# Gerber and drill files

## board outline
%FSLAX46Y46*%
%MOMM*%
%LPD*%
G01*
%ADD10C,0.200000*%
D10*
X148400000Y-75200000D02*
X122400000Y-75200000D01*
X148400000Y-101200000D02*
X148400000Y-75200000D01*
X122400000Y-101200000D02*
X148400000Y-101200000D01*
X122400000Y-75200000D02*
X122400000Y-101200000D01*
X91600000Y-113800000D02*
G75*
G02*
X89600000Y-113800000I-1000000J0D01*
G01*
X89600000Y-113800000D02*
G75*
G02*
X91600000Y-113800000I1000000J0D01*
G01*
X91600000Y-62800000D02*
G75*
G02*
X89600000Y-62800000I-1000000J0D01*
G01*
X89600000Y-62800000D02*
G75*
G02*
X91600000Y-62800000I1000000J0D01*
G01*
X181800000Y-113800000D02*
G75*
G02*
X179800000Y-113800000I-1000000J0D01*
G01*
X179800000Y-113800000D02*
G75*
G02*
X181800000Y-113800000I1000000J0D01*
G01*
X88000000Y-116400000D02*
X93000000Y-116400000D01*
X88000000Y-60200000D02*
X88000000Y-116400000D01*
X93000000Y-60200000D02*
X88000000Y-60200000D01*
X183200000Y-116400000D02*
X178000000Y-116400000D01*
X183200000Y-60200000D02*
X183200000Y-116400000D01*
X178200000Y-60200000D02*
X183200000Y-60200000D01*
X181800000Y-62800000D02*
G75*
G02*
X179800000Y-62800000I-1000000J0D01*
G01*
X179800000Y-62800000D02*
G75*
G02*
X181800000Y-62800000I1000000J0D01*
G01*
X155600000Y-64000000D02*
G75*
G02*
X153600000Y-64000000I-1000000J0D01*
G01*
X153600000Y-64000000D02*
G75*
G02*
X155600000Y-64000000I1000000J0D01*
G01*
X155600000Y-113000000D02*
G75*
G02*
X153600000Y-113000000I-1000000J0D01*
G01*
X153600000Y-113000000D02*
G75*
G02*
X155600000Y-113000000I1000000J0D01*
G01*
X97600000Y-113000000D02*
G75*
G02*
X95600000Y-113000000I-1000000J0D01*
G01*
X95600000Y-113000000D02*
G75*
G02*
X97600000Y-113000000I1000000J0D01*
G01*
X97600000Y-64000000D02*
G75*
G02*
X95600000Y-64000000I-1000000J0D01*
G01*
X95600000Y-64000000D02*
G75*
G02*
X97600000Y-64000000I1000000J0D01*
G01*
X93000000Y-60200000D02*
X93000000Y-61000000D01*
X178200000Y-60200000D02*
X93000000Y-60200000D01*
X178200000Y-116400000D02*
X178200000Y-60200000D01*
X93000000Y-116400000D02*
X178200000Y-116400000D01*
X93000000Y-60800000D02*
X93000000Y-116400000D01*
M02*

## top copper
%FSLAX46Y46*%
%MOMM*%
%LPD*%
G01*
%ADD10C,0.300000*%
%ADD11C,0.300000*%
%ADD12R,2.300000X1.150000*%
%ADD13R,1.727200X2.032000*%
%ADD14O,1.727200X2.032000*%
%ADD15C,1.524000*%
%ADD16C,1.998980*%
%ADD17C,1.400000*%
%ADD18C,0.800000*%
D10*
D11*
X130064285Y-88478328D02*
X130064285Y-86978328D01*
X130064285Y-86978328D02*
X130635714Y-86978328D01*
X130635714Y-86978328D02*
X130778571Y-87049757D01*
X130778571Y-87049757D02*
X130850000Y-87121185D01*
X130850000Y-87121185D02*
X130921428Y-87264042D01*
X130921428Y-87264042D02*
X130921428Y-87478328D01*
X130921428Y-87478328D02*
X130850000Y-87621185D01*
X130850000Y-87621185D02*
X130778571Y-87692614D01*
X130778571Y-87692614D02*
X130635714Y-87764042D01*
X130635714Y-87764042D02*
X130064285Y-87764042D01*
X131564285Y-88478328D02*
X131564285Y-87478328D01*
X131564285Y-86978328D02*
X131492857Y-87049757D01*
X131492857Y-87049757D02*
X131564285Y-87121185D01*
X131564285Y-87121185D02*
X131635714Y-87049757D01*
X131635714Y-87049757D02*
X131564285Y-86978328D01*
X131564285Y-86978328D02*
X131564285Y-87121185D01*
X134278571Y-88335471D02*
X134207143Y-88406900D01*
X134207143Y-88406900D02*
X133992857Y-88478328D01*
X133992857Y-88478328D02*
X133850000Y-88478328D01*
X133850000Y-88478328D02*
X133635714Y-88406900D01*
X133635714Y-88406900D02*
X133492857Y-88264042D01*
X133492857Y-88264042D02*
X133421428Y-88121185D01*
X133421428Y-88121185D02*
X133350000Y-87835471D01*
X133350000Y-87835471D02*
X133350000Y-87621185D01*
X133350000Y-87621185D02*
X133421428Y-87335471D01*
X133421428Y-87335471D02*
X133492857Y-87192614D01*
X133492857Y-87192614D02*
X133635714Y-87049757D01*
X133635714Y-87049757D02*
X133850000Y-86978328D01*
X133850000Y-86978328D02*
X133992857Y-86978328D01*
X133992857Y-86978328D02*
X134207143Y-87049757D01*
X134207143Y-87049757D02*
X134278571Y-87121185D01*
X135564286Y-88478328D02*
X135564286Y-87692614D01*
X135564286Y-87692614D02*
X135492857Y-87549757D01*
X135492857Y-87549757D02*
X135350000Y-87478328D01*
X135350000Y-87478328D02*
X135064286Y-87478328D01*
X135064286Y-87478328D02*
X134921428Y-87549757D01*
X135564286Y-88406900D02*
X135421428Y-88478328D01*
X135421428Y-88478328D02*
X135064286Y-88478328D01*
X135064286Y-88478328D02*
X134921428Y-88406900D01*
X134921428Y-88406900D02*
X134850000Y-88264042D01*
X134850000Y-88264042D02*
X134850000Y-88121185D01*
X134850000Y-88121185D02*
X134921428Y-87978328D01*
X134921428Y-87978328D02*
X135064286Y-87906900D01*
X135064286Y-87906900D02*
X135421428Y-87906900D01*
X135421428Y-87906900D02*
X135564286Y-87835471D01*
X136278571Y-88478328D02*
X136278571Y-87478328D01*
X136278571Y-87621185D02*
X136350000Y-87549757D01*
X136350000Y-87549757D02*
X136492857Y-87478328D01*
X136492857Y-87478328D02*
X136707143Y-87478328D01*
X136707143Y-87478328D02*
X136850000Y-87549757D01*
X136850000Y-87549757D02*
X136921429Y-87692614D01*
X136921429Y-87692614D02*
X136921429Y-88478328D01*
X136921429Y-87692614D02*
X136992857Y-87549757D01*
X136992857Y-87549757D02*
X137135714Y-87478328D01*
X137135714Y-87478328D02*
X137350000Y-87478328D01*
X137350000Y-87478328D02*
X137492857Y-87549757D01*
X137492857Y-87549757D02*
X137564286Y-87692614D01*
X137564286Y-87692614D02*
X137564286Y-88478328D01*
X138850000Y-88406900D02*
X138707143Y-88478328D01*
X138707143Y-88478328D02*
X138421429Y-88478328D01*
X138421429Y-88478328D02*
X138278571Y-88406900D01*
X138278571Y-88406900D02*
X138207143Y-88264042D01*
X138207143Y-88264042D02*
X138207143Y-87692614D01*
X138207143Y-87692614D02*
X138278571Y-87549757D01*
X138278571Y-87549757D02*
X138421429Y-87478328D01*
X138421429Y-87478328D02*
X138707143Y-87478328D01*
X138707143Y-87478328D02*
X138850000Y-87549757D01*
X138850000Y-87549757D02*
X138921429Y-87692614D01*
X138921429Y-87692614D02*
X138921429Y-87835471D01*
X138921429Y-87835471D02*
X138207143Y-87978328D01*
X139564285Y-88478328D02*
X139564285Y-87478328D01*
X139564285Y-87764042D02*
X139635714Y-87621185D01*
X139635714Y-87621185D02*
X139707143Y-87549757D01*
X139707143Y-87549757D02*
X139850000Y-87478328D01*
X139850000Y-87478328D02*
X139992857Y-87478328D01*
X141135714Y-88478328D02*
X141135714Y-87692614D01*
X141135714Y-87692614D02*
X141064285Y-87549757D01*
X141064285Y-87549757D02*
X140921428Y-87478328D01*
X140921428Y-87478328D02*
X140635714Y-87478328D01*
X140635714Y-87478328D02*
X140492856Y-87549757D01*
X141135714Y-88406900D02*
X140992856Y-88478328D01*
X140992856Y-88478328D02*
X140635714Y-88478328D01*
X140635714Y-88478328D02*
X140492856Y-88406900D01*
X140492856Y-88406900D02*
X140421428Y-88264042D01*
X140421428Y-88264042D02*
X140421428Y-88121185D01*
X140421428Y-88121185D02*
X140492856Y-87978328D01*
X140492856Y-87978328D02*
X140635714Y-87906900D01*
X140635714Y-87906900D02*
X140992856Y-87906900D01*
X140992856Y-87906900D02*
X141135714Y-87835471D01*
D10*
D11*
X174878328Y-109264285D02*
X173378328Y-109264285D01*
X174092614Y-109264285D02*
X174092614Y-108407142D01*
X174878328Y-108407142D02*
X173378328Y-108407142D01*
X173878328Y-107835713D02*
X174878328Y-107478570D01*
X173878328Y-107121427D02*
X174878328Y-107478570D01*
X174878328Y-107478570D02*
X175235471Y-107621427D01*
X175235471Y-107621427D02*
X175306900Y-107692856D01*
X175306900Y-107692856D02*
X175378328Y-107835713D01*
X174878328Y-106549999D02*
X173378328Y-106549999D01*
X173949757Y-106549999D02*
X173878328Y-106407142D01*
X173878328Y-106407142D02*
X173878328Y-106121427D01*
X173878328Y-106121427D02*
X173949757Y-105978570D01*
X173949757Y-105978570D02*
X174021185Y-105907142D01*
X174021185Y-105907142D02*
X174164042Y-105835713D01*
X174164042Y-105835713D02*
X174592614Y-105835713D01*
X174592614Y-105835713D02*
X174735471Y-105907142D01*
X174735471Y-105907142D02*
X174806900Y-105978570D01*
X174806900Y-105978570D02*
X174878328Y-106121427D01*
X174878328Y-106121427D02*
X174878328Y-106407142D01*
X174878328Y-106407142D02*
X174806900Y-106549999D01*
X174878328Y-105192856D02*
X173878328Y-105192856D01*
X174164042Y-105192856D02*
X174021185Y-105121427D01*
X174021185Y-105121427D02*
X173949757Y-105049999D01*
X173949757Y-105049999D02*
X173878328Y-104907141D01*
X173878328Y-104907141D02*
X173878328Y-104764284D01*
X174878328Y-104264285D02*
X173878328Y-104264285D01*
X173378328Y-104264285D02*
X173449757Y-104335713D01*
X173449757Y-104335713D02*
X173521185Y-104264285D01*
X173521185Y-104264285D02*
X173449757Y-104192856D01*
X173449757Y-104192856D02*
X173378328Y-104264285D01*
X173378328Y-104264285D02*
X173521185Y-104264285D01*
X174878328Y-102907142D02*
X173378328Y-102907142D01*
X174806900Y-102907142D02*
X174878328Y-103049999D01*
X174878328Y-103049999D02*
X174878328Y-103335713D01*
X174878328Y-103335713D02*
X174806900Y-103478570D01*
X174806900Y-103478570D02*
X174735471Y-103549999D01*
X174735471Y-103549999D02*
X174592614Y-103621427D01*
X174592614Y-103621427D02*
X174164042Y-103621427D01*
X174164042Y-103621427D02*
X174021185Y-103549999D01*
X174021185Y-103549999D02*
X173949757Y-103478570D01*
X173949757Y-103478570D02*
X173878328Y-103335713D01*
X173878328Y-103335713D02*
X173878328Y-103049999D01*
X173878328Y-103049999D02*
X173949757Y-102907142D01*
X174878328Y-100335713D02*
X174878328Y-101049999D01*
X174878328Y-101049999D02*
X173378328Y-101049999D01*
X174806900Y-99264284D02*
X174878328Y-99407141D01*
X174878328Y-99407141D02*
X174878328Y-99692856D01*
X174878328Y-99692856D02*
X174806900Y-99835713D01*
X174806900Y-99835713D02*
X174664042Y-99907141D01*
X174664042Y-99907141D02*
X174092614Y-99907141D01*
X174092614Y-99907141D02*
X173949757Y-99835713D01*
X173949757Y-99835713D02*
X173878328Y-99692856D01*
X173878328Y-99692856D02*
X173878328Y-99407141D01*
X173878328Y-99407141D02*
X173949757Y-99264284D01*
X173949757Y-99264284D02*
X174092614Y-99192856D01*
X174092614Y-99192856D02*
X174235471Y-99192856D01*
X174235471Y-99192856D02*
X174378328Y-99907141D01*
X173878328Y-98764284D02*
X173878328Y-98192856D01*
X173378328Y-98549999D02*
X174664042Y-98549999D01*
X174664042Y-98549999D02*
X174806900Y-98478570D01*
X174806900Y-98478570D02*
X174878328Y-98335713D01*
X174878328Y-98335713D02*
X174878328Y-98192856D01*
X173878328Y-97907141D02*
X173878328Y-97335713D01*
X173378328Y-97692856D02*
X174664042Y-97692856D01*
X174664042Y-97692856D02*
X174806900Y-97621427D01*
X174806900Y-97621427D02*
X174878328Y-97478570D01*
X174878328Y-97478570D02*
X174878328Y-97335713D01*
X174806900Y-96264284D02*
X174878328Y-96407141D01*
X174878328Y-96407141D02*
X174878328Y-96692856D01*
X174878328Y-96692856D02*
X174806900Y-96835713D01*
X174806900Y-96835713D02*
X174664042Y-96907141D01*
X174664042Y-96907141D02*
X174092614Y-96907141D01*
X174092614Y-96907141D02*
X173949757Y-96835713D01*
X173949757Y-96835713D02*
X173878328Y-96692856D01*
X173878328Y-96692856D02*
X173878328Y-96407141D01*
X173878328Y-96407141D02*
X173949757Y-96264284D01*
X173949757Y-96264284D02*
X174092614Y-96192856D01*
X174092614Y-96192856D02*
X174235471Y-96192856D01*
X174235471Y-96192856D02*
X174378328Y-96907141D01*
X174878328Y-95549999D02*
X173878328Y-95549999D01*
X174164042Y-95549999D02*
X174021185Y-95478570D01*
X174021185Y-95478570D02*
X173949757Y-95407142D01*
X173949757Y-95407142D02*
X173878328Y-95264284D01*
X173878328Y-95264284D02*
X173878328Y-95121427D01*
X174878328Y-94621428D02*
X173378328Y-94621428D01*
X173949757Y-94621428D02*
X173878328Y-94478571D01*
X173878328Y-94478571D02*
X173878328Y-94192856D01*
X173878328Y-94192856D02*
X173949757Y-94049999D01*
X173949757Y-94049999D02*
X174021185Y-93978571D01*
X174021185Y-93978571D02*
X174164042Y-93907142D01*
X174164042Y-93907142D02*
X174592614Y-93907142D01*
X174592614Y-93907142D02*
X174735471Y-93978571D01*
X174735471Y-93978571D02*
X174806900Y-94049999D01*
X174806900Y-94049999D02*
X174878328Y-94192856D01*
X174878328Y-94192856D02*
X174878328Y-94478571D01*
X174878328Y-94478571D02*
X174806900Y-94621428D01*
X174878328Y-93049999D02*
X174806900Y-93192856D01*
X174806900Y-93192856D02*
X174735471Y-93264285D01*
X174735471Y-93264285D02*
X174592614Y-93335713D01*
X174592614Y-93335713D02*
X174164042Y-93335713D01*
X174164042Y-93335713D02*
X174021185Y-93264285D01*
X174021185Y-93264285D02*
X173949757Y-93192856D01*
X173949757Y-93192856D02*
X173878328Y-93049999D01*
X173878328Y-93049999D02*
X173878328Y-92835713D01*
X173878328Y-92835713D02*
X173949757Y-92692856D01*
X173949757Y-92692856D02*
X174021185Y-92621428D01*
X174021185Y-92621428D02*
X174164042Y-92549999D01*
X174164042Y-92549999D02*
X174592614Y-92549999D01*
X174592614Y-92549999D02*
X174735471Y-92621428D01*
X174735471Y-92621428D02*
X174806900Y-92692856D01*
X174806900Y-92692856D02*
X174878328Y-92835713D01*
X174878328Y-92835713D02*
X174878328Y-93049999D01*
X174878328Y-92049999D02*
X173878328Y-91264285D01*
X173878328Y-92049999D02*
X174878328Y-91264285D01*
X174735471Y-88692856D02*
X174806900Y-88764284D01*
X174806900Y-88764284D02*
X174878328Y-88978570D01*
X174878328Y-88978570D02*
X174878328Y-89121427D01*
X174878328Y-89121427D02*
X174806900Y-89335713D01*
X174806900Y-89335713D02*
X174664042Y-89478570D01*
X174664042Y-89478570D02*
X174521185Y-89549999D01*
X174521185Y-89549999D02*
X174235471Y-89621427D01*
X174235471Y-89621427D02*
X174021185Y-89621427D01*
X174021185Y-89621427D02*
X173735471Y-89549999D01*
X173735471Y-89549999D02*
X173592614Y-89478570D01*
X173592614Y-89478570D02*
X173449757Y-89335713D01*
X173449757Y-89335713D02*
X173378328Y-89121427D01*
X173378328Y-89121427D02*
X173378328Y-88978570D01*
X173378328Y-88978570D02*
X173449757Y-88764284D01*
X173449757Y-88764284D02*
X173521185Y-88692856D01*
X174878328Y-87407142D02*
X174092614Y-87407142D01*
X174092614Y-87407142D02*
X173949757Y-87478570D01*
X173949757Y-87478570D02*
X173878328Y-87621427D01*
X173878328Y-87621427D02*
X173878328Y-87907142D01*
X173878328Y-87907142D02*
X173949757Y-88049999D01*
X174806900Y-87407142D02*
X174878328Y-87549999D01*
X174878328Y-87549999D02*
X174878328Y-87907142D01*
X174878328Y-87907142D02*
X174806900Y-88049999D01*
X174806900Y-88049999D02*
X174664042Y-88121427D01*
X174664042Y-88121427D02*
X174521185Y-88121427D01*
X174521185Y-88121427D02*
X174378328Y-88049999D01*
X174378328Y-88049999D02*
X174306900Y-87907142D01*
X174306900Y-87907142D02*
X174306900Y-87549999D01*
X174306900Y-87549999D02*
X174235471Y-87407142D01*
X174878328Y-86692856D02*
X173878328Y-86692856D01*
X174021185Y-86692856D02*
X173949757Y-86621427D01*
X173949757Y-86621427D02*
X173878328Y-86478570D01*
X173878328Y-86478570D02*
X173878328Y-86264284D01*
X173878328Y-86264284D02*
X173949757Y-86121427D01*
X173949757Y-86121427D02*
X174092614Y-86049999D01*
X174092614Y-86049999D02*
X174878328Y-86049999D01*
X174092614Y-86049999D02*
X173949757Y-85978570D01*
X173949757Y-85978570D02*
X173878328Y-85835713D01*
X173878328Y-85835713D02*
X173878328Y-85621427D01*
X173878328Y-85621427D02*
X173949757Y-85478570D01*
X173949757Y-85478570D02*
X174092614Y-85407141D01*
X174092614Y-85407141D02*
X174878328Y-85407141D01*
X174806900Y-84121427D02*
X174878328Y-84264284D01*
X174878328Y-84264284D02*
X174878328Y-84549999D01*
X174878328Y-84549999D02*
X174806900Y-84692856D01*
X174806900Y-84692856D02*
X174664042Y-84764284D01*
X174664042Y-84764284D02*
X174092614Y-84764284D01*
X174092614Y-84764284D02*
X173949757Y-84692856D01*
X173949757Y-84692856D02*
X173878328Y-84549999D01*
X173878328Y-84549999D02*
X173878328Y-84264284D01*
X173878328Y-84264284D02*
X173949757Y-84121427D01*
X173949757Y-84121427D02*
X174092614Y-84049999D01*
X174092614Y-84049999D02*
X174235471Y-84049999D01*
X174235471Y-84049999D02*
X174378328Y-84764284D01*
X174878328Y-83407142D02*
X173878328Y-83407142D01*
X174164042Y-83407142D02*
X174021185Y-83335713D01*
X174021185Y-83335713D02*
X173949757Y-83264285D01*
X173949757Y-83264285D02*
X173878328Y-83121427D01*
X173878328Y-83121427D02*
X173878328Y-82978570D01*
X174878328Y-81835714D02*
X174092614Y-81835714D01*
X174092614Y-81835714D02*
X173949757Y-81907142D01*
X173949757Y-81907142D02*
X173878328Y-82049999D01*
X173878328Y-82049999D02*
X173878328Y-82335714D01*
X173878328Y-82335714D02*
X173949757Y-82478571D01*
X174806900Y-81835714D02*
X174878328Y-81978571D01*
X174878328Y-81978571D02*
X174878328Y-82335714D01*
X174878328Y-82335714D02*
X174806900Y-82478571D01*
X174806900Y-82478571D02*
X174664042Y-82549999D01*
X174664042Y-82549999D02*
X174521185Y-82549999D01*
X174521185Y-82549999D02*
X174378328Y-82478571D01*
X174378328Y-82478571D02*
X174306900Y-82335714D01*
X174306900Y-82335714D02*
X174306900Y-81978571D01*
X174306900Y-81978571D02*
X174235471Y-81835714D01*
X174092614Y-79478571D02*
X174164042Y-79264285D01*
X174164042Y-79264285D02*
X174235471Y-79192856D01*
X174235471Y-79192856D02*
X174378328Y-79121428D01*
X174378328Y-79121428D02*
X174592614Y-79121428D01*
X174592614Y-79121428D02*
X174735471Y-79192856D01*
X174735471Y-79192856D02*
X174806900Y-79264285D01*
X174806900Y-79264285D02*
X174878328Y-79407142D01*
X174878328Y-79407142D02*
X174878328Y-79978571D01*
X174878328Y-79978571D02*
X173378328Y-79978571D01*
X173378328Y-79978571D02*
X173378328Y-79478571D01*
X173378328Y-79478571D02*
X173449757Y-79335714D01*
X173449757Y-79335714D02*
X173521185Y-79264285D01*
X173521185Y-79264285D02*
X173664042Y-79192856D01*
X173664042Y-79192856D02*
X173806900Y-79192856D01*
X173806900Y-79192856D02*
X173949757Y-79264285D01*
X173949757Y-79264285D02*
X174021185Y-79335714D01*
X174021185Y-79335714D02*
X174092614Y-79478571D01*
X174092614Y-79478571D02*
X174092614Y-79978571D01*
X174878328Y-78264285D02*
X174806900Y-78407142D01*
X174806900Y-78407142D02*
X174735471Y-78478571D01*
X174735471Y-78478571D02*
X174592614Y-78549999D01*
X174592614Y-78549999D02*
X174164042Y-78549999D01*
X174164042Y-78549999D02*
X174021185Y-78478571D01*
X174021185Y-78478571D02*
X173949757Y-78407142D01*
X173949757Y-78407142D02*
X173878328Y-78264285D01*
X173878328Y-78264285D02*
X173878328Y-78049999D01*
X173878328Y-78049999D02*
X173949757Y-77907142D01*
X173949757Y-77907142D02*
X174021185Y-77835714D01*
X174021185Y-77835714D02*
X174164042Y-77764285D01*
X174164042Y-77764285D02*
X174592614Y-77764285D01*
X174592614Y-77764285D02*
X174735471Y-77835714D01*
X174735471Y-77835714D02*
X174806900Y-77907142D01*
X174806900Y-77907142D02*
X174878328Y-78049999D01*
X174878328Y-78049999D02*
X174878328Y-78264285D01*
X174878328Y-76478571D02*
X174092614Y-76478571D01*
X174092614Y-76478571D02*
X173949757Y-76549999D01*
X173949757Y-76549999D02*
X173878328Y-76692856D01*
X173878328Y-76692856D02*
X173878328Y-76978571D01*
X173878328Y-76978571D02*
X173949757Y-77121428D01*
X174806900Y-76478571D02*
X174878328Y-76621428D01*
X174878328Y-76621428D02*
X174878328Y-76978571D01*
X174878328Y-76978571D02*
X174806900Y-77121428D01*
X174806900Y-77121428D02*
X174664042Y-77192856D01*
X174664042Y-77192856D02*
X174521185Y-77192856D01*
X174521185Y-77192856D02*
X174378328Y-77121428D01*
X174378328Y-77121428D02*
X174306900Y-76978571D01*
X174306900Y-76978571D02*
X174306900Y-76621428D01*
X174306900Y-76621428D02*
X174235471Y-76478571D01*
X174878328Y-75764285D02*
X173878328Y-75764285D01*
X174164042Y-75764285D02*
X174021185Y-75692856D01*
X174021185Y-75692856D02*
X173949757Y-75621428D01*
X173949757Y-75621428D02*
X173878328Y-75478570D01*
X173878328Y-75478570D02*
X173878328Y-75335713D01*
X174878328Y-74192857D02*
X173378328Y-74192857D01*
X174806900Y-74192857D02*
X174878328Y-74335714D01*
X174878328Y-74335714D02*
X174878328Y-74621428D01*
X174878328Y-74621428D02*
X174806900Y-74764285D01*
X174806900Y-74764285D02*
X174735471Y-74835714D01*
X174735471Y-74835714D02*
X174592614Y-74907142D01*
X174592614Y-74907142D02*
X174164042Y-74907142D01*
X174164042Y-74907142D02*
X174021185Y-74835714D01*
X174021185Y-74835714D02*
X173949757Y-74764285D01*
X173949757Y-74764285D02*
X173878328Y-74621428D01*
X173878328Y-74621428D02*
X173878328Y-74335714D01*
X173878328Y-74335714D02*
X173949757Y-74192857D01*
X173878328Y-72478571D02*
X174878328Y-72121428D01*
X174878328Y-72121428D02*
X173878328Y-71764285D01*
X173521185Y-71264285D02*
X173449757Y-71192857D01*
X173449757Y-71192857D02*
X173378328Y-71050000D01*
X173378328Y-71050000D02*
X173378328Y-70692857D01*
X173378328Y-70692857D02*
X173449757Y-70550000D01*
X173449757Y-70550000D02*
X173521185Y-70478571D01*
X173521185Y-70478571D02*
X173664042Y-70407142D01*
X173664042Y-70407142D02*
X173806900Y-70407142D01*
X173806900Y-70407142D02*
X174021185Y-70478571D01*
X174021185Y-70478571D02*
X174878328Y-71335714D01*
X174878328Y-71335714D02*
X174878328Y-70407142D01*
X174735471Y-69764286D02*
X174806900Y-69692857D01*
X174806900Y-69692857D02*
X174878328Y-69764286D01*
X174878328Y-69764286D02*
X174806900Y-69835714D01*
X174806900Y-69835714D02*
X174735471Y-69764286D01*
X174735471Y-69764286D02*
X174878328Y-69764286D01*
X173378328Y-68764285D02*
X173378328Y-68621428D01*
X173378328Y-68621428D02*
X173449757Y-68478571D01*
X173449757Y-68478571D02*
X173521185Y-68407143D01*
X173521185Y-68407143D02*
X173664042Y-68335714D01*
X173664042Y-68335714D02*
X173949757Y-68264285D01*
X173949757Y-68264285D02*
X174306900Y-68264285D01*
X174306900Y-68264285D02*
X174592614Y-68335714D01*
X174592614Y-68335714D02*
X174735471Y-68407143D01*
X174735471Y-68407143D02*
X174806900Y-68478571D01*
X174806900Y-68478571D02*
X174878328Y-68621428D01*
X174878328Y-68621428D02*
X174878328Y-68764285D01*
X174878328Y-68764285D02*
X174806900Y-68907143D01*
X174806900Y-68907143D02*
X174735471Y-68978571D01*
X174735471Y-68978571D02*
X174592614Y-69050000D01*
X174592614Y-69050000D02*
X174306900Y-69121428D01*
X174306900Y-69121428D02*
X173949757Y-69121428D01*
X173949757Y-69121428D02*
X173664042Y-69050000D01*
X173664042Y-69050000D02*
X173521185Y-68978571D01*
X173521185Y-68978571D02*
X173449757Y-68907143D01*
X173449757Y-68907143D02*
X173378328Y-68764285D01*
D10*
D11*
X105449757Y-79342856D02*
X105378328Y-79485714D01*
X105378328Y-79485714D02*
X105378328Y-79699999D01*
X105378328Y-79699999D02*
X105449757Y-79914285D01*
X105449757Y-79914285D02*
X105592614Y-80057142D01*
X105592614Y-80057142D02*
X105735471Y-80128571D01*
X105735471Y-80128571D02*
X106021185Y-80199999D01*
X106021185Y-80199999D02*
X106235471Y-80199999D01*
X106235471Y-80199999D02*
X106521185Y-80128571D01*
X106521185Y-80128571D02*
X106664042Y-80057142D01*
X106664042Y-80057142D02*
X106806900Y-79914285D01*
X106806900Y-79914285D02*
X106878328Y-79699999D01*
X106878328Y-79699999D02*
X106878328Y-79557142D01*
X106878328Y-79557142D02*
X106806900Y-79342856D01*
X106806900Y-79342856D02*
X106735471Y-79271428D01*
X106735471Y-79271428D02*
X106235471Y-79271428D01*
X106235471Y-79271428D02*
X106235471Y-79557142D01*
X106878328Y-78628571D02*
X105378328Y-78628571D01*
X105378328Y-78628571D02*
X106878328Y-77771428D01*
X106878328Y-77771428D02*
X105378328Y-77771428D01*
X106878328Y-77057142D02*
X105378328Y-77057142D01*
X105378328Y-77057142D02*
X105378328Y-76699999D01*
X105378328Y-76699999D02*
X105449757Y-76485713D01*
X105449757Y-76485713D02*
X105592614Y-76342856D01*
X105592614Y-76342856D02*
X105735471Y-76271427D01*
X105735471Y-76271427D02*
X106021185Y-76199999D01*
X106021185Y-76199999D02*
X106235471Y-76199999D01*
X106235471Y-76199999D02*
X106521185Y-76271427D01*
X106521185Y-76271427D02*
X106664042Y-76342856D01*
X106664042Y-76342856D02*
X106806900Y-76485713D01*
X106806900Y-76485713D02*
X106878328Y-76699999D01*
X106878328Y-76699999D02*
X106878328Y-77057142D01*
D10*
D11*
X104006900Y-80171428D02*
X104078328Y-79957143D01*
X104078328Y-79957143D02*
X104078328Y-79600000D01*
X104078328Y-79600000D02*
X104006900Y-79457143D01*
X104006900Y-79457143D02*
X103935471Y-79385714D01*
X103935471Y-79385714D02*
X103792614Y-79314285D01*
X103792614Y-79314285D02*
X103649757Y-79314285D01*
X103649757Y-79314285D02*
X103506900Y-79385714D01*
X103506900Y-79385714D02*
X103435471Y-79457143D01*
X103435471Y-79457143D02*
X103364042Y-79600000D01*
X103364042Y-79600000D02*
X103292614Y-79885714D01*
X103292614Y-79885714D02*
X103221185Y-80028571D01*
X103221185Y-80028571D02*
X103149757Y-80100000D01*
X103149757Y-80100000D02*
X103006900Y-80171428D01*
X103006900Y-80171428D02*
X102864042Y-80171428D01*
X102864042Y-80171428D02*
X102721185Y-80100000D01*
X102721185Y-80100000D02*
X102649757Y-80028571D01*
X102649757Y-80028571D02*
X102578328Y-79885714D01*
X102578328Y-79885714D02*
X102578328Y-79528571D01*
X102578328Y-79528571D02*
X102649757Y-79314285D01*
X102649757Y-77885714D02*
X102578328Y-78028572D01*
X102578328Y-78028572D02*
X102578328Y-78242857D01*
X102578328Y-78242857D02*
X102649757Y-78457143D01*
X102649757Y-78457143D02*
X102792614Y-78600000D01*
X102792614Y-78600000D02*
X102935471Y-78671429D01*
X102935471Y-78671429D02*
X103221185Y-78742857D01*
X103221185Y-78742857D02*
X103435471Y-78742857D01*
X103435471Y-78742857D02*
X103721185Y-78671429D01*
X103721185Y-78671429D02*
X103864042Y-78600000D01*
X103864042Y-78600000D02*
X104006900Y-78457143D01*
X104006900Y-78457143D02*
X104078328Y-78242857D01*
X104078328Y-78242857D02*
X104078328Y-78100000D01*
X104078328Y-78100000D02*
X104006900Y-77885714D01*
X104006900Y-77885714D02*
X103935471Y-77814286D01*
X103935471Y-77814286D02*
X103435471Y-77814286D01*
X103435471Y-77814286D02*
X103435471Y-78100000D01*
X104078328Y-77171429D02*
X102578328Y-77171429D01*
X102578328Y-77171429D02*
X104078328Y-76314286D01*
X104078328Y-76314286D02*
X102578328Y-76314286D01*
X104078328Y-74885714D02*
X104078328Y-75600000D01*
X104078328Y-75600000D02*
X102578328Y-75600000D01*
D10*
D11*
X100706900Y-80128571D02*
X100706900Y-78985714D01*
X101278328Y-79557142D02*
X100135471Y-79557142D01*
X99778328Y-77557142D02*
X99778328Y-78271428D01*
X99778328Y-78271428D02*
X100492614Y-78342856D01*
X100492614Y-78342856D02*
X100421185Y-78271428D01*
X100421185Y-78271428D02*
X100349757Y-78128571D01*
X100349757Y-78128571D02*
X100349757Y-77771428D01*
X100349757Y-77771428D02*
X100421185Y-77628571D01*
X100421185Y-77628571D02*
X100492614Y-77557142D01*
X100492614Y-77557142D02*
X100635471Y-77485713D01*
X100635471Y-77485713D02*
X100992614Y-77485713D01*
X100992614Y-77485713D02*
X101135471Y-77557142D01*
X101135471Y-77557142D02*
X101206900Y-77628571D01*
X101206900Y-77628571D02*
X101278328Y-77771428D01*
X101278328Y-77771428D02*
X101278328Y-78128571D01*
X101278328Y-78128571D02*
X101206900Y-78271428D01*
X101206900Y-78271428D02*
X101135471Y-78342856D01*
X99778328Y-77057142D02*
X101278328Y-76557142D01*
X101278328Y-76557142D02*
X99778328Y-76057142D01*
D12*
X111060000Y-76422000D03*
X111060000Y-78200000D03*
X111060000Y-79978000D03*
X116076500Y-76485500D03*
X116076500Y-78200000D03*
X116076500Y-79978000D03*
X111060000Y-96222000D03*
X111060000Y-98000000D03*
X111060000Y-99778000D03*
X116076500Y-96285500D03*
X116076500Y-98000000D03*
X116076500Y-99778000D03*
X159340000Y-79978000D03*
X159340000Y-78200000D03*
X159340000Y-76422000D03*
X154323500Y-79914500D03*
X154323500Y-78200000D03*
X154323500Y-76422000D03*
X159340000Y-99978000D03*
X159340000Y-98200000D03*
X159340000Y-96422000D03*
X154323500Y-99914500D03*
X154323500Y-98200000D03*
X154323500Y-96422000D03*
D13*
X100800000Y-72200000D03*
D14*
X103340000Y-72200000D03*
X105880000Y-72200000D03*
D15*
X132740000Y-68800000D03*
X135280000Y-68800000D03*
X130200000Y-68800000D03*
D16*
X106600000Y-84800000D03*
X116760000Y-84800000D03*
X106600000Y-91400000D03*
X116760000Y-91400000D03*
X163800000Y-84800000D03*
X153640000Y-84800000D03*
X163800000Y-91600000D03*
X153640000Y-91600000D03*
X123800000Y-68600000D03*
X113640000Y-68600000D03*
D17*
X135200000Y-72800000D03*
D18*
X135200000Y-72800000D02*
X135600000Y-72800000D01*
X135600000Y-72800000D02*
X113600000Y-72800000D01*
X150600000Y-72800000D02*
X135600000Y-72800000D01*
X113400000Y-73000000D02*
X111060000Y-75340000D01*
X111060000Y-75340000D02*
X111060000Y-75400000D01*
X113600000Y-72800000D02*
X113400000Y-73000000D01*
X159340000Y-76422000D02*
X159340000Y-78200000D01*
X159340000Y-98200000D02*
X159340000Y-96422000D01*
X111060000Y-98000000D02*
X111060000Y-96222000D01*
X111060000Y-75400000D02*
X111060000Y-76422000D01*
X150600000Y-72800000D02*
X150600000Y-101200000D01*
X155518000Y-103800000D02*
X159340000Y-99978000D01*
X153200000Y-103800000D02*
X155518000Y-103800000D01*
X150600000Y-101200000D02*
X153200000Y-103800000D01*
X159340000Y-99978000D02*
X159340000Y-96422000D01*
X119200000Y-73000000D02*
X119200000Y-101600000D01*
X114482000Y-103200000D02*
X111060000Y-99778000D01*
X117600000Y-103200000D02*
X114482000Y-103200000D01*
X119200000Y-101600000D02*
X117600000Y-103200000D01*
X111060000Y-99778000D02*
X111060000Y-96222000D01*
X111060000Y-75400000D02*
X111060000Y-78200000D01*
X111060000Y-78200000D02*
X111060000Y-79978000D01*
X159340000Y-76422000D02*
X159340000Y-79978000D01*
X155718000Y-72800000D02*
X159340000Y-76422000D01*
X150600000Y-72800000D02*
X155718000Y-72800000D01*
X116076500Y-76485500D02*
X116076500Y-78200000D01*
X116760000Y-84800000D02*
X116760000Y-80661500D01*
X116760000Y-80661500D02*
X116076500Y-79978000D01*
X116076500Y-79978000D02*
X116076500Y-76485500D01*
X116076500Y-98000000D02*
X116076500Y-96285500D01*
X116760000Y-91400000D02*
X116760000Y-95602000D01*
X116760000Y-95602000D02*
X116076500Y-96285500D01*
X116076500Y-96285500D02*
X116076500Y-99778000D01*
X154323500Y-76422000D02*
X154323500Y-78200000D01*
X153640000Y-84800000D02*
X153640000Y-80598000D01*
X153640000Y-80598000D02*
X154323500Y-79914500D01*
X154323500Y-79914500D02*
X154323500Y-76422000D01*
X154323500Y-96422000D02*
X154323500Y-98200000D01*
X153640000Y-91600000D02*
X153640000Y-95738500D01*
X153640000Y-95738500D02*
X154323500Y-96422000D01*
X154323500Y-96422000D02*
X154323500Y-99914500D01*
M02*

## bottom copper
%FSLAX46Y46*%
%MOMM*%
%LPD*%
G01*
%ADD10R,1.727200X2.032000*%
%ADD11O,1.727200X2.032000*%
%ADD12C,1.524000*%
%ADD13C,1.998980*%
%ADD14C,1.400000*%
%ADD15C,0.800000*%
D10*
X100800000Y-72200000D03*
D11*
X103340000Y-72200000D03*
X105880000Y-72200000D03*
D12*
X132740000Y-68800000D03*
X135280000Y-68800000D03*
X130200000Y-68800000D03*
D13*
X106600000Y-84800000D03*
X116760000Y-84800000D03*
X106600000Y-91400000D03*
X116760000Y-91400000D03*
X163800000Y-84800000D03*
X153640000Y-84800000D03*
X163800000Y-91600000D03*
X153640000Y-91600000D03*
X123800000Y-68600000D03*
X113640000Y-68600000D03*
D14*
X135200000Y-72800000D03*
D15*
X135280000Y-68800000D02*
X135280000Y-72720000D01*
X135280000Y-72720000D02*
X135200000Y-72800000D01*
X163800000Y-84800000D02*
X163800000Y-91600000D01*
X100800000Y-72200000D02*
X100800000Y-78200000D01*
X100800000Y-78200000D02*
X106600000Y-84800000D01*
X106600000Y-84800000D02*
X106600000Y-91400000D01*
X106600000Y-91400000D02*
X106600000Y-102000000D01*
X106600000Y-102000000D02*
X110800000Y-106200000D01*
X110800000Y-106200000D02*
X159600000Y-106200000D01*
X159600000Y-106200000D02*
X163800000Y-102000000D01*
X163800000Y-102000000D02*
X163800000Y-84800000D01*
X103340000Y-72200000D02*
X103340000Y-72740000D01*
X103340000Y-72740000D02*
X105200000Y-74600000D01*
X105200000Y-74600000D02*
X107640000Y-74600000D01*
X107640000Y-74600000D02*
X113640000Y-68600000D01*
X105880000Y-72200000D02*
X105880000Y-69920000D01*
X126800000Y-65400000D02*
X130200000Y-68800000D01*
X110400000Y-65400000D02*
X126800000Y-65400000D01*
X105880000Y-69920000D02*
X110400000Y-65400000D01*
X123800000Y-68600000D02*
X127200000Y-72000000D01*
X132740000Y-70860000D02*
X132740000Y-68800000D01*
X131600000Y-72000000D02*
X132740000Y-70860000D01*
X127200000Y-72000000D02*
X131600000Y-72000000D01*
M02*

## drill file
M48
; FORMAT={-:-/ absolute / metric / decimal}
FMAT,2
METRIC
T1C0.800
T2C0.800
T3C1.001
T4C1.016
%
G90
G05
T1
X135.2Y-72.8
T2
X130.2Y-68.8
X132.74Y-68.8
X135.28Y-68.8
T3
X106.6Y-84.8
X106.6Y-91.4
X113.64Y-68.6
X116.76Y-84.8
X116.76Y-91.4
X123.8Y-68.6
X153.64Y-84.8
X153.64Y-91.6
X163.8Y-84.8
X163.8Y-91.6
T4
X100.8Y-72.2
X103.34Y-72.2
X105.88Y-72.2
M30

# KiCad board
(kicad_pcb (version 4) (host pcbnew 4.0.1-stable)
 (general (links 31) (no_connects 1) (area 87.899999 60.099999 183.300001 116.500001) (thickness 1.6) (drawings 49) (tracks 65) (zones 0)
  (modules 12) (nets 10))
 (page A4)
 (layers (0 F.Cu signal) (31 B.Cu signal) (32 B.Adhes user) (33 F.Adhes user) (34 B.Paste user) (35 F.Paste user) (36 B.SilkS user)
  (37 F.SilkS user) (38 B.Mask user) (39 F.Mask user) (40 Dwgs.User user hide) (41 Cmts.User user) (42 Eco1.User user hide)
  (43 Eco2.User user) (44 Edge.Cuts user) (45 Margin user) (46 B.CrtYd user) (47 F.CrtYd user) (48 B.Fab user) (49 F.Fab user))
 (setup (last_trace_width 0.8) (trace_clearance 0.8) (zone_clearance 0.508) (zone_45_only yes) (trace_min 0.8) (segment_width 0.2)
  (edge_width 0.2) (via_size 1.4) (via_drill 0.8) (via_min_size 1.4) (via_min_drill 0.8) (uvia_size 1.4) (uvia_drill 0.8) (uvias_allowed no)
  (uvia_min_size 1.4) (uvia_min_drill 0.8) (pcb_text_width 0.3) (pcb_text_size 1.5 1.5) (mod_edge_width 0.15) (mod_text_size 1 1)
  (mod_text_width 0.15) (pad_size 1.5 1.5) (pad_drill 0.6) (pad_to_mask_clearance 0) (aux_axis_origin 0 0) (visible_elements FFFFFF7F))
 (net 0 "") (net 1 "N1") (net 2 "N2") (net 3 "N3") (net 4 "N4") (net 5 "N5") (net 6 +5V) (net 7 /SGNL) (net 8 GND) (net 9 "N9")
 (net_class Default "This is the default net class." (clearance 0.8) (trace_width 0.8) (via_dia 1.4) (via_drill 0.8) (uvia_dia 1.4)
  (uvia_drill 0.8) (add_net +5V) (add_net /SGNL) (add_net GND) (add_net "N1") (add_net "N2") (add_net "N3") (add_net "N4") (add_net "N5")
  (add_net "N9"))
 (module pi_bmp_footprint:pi (layer F.Cu) (at 135.4 88.2)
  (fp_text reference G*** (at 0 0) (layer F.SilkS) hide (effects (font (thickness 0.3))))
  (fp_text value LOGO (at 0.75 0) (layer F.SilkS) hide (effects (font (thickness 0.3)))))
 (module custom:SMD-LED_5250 (layer F.Cu) (at 113.6 78.2)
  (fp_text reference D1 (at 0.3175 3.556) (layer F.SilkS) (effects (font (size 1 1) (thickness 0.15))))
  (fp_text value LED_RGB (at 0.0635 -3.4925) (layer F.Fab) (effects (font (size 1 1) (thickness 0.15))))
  (pad 1 smd rect (at -2.54 -1.778) (size 2.3 1.15) (layers F.Cu F.Paste F.Mask) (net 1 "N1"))
  (pad 2 smd rect (at -2.54 0) (size 2.3 1.15) (layers F.Cu F.Paste F.Mask) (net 1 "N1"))
  (pad 3 smd rect (at -2.54 1.778) (size 2.3 1.15) (layers F.Cu F.Paste F.Mask) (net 1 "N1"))
  (pad 4 smd rect (at 2.4765 -1.7145) (size 2.3 1.15) (layers F.Cu F.Paste F.Mask) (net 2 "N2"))
  (pad 5 smd rect (at 2.4765 0) (size 2.3 1.15) (layers F.Cu F.Paste F.Mask) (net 2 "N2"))
  (pad 6 smd rect (at 2.4765 1.778) (size 2.3 1.15) (layers F.Cu F.Paste F.Mask) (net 2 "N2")))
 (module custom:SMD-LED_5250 (layer F.Cu) (at 113.6 98)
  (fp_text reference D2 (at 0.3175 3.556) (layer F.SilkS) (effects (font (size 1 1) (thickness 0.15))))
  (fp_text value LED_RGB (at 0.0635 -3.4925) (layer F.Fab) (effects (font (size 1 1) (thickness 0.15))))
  (pad 1 smd rect (at -2.54 -1.778) (size 2.3 1.15) (layers F.Cu F.Paste F.Mask) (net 1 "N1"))
  (pad 2 smd rect (at -2.54 0) (size 2.3 1.15) (layers F.Cu F.Paste F.Mask) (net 1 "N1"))
  (pad 3 smd rect (at -2.54 1.778) (size 2.3 1.15) (layers F.Cu F.Paste F.Mask) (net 1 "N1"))
  (pad 4 smd rect (at 2.4765 -1.7145) (size 2.3 1.15) (layers F.Cu F.Paste F.Mask) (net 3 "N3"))
  (pad 5 smd rect (at 2.4765 0) (size 2.3 1.15) (layers F.Cu F.Paste F.Mask) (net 3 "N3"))
  (pad 6 smd rect (at 2.4765 1.778) (size 2.3 1.15) (layers F.Cu F.Paste F.Mask) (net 3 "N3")))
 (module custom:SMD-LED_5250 (layer F.Cu) (at 156.8 78.2 180)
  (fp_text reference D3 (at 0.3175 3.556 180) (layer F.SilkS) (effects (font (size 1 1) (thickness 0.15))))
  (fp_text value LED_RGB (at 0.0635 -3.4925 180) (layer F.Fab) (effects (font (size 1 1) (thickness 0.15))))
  (pad 1 smd rect (at -2.54 -1.778 180) (size 2.3 1.15) (layers F.Cu F.Paste F.Mask) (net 1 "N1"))
  (pad 2 smd rect (at -2.54 0 180) (size 2.3 1.15) (layers F.Cu F.Paste F.Mask) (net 1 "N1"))
  (pad 3 smd rect (at -2.54 1.778 180) (size 2.3 1.15) (layers F.Cu F.Paste F.Mask) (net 1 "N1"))
  (pad 4 smd rect (at 2.4765 -1.7145 180) (size 2.3 1.15) (layers F.Cu F.Paste F.Mask) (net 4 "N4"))
  (pad 5 smd rect (at 2.4765 0 180) (size 2.3 1.15) (layers F.Cu F.Paste F.Mask) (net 4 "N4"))
  (pad 6 smd rect (at 2.4765 1.778 180) (size 2.3 1.15) (layers F.Cu F.Paste F.Mask) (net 4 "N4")))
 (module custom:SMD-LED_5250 (layer F.Cu) (at 156.8 98.2 180)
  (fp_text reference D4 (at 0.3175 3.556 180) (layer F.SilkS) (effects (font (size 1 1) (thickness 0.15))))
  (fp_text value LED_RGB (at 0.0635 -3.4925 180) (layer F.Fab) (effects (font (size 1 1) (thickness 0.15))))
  (pad 1 smd rect (at -2.54 -1.778 180) (size 2.3 1.15) (layers F.Cu F.Paste F.Mask) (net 1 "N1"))
  (pad 2 smd rect (at -2.54 0 180) (size 2.3 1.15) (layers F.Cu F.Paste F.Mask) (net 1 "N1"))
  (pad 3 smd rect (at -2.54 1.778 180) (size 2.3 1.15) (layers F.Cu F.Paste F.Mask) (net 1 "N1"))
  (pad 4 smd rect (at 2.4765 -1.7145 180) (size 2.3 1.15) (layers F.Cu F.Paste F.Mask) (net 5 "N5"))
  (pad 5 smd rect (at 2.4765 0 180) (size 2.3 1.15) (layers F.Cu F.Paste F.Mask) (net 5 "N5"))
  (pad 6 smd rect (at 2.4765 1.778 180) (size 2.3 1.15) (layers F.Cu F.Paste F.Mask) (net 5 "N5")))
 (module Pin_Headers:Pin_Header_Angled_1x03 (layer F.Cu) (at 100.8 72.2 90)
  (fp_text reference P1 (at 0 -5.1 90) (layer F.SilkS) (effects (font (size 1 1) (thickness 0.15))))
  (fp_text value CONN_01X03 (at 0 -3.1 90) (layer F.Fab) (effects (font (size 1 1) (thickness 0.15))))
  (pad 1 thru_hole rect (at 0 0 90) (size 2.032 1.7272) (drill 1.016) (layers *.Cu *.Mask F.SilkS) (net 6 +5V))
  (pad 2 thru_hole oval (at 0 2.54 90) (size 2.032 1.7272) (drill 1.016) (layers *.Cu *.Mask F.SilkS) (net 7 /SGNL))
  (pad 3 thru_hole oval (at 0 5.08 90) (size 2.032 1.7272) (drill 1.016) (layers *.Cu *.Mask F.SilkS) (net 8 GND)))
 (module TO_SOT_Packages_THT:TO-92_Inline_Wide (layer F.Cu) (at 130.2 68.8)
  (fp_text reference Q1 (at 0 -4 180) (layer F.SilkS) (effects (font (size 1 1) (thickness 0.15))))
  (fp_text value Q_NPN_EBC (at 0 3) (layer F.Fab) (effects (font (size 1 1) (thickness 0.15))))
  (pad 2 thru_hole circle (at 2.54 0 90) (size 1.524 1.524) (drill 0.8) (layers *.Cu *.Mask F.SilkS) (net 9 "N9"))
  (pad 3 thru_hole circle (at 5.08 0 90) (size 1.524 1.524) (drill 0.8) (layers *.Cu *.Mask F.SilkS) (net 1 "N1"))
  (pad 1 thru_hole circle (at 0 0 90) (size 1.524 1.524) (drill 0.8) (layers *.Cu *.Mask F.SilkS) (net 8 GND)))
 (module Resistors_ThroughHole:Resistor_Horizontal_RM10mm (layer F.Cu) (at 106.6 84.8)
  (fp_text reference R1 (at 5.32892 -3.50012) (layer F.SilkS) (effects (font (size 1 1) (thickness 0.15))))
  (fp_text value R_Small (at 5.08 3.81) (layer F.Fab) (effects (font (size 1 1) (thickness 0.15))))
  (pad 1 thru_hole circle (at 0 0) (size 1.99898 1.99898) (drill 1.00076) (layers *.Cu *.SilkS *.Mask) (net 6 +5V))
  (pad 2 thru_hole circle (at 10.16 0) (size 1.99898 1.99898) (drill 1.00076) (layers *.Cu *.SilkS *.Mask) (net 2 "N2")))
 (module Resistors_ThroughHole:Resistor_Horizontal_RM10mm (layer F.Cu) (at 106.6 91.4)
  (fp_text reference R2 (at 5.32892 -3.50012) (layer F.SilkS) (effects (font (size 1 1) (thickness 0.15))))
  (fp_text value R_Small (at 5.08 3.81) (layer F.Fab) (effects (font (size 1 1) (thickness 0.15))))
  (pad 1 thru_hole circle (at 0 0) (size 1.99898 1.99898) (drill 1.00076) (layers *.Cu *.SilkS *.Mask) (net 6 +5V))
  (pad 2 thru_hole circle (at 10.16 0) (size 1.99898 1.99898) (drill 1.00076) (layers *.Cu *.SilkS *.Mask) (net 3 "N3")))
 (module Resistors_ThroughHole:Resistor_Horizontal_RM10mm (layer F.Cu) (at 163.8 84.8 180)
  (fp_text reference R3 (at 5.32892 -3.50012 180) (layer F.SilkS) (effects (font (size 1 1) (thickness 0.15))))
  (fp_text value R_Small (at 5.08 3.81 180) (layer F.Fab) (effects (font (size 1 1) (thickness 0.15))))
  (pad 1 thru_hole circle (at 0 0 180) (size 1.99898 1.99898) (drill 1.00076) (layers *.Cu *.SilkS *.Mask) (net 6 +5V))
  (pad 2 thru_hole circle (at 10.16 0 180) (size 1.99898 1.99898) (drill 1.00076) (layers *.Cu *.SilkS *.Mask) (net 4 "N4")))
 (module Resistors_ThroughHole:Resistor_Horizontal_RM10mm (layer F.Cu) (at 163.8 91.6 180)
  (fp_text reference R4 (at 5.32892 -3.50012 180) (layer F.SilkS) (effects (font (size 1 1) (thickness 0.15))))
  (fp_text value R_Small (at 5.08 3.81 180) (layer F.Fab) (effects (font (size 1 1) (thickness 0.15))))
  (pad 1 thru_hole circle (at 0 0 180) (size 1.99898 1.99898) (drill 1.00076) (layers *.Cu *.SilkS *.Mask) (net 6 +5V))
  (pad 2 thru_hole circle (at 10.16 0 180) (size 1.99898 1.99898) (drill 1.00076) (layers *.Cu *.SilkS *.Mask) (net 5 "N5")))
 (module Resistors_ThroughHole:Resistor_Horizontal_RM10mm (layer F.Cu) (at 123.8 68.6 180)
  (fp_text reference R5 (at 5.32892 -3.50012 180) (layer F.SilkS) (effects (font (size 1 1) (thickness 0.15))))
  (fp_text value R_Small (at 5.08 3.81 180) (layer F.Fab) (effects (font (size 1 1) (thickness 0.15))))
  (pad 1 thru_hole circle (at 0 0 180) (size 1.99898 1.99898) (drill 1.00076) (layers *.Cu *.SilkS *.Mask) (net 9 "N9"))
  (pad 2 thru_hole circle (at 10.16 0 180) (size 1.99898 1.99898) (drill 1.00076) (layers *.Cu *.SilkS *.Mask) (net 7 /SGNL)))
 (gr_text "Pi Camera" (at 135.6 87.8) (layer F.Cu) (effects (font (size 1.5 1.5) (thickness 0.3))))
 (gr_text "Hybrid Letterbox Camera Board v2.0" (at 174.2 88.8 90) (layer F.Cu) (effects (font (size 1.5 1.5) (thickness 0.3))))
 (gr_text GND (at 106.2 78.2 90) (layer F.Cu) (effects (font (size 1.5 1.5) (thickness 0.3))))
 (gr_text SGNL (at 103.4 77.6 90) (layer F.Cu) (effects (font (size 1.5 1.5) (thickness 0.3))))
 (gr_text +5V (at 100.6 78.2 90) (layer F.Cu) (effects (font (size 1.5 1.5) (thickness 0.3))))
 (gr_line (start 148.4 75.2) (end 122.4 75.2) (angle 90) (layer Edge.Cuts) (width 0.2))
 (gr_line (start 148.4 101.2) (end 148.4 75.2) (angle 90) (layer Edge.Cuts) (width 0.2))
 (gr_line (start 122.4 101.2) (end 148.4 101.2) (angle 90) (layer Edge.Cuts) (width 0.2))
 (gr_line (start 122.4 75.2) (end 122.4 101.2) (angle 90) (layer Edge.Cuts) (width 0.2))
 (gr_circle (center 90.6 113.8) (end 91.4 114.4) (layer Edge.Cuts) (width 0.2))
 (gr_circle (center 90.6 62.8) (end 91.4 63.4) (layer Edge.Cuts) (width 0.2))
 (gr_circle (center 180.8 113.8) (end 181.6 114.4) (layer Edge.Cuts) (width 0.2))
 (gr_line (start 88 116.4) (end 93 116.4) (angle 90) (layer Edge.Cuts) (width 0.2))
 (gr_line (start 88 60.2) (end 88 116.4) (angle 90) (layer Edge.Cuts) (width 0.2))
 (gr_line (start 93 60.2) (end 88 60.2) (angle 90) (layer Edge.Cuts) (width 0.2))
 (gr_line (start 183.2 116.4) (end 178 116.4) (angle 90) (layer Edge.Cuts) (width 0.2))
 (gr_line (start 183.2 60.2) (end 183.2 116.4) (angle 90) (layer Edge.Cuts) (width 0.2))
 (gr_line (start 178.2 60.2) (end 183.2 60.2) (angle 90) (layer Edge.Cuts) (width 0.2))
 (gr_circle (center 180.8 62.8) (end 181.6 63.4) (layer Edge.Cuts) (width 0.2))
 (gr_circle (center 154.6 64) (end 155.4 64.6) (layer Edge.Cuts) (width 0.2))
 (gr_circle (center 154.6 113) (end 155.4 113.6) (layer Edge.Cuts) (width 0.2))
 (gr_circle (center 96.6 113) (end 97.4 113.6) (layer Edge.Cuts) (width 0.2))
 (gr_circle (center 96.6 64) (end 97.4 64.6) (layer Edge.Cuts) (width 0.2))
 (gr_line (start 93 60.2) (end 93 61) (angle 90) (layer Edge.Cuts) (width 0.2))
 (gr_line (start 178.2 60.2) (end 93 60.2) (angle 90) (layer Edge.Cuts) (width 0.2))
 (gr_line (start 178.2 116.4) (end 178.2 60.2) (angle 90) (layer Edge.Cuts) (width 0.2))
 (gr_line (start 93 116.4) (end 178.2 116.4) (angle 90) (layer Edge.Cuts) (width 0.2))
 (gr_line (start 93 60.8) (end 93 116.4) (angle 90) (layer Edge.Cuts) (width 0.2))
 (segment (start 135.28 68.8) (end 135.28 72.72) (width 0.8) (layer B.Cu) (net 1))
 (segment (start 135.2 72.8) (end 135.6 72.8) (width 0.8) (layer F.Cu) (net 1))
 (via (at 135.2 72.8) (size 1.4) (drill 0.8) (layers F.Cu B.Cu) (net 1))
 (segment (start 135.28 72.72) (end 135.2 72.8) (width 0.8) (layer B.Cu) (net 1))
 (segment (start 135.6 72.8) (end 113.6 72.8) (width 0.8) (layer F.Cu) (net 1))
 (segment (start 150.6 72.8) (end 135.6 72.8) (width 0.8) (layer F.Cu) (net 1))
 (segment (start 113.4 73) (end 111.06 75.34) (width 0.8) (layer F.Cu) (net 1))
 (segment (start 111.06 75.34) (end 111.06 75.4) (width 0.8) (layer F.Cu) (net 1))
 (segment (start 113.6 72.8) (end 113.4 73) (width 0.8) (layer F.Cu) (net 1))
 (segment (start 159.34 76.422) (end 159.34 78.2) (width 0.8) (layer F.Cu) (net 1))
 (segment (start 159.34 98.2) (end 159.34 96.422) (width 0.8) (layer F.Cu) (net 1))
 (segment (start 111.06 98) (end 111.06 96.222) (width 0.8) (layer F.Cu) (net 1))
 (segment (start 111.06 75.4) (end 111.06 76.422) (width 0.8) (layer F.Cu) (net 1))
 (segment (start 150.6 72.8) (end 150.6 101.2) (width 0.8) (layer F.Cu) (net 1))
 (segment (start 155.518 103.8) (end 159.34 99.978) (width 0.8) (layer F.Cu) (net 1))
 (segment (start 153.2 103.8) (end 155.518 103.8) (width 0.8) (layer F.Cu) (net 1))
 (segment (start 150.6 101.2) (end 153.2 103.8) (width 0.8) (layer F.Cu) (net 1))
 (segment (start 159.34 99.978) (end 159.34 96.422) (width 0.8) (layer F.Cu) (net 1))
 (segment (start 119.2 73) (end 119.2 101.6) (width 0.8) (layer F.Cu) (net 1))
 (segment (start 114.482 103.2) (end 111.06 99.778) (width 0.8) (layer F.Cu) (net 1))
 (segment (start 117.6 103.2) (end 114.482 103.2) (width 0.8) (layer F.Cu) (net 1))
 (segment (start 119.2 101.6) (end 117.6 103.2) (width 0.8) (layer F.Cu) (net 1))
 (segment (start 111.06 99.778) (end 111.06 96.222) (width 0.8) (layer F.Cu) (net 1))
 (segment (start 111.06 75.4) (end 111.06 78.2) (width 0.8) (layer F.Cu) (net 1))
 (segment (start 111.06 78.2) (end 111.06 79.978) (width 0.8) (layer F.Cu) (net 1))
 (segment (start 159.34 76.422) (end 159.34 79.978) (width 0.8) (layer F.Cu) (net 1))
 (segment (start 155.718 72.8) (end 159.34 76.422) (width 0.8) (layer F.Cu) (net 1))
 (segment (start 150.6 72.8) (end 155.718 72.8) (width 0.8) (layer F.Cu) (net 1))
 (segment (start 116.0765 76.4855) (end 116.0765 78.2) (width 0.8) (layer F.Cu) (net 2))
 (segment (start 116.76 84.8) (end 116.76 80.6615) (width 0.8) (layer F.Cu) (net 2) (status 10))
 (segment (start 116.76 80.6615) (end 116.0765 79.978) (width 0.8) (layer F.Cu) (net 2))
 (segment (start 116.0765 79.978) (end 116.0765 76.4855) (width 0.8) (layer F.Cu) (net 2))
 (segment (start 116.0765 98) (end 116.0765 96.2855) (width 0.8) (layer F.Cu) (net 3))
 (segment (start 116.76 91.4) (end 116.76 95.602) (width 0.8) (layer F.Cu) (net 3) (status 10))
 (segment (start 116.76 95.602) (end 116.0765 96.2855) (width 0.8) (layer F.Cu) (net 3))
 (segment (start 116.0765 96.2855) (end 116.0765 99.778) (width 0.8) (layer F.Cu) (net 3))
 (segment (start 154.3235 76.422) (end 154.3235 78.2) (width 0.8) (layer F.Cu) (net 4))
 (segment (start 153.64 84.8) (end 153.64 80.598) (width 0.8) (layer F.Cu) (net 4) (status 10))
 (segment (start 153.64 80.598) (end 154.3235 79.9145) (width 0.8) (layer F.Cu) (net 4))
 (segment (start 154.3235 79.9145) (end 154.3235 76.422) (width 0.8) (layer F.Cu) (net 4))
 (segment (start 154.3235 96.422) (end 154.3235 98.2) (width 0.8) (layer F.Cu) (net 5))
 (segment (start 153.64 91.6) (end 153.64 95.7385) (width 0.8) (layer F.Cu) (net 5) (status 10))
 (segment (start 153.64 95.7385) (end 154.3235 96.422) (width 0.8) (layer F.Cu) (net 5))
 (segment (start 154.3235 96.422) (end 154.3235 99.9145) (width 0.8) (layer F.Cu) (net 5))
 (segment (start 163.8 84.8) (end 163.8 91.6) (width 0.8) (layer B.Cu) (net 6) (status 20))
 (segment (start 100.8 72.2) (end 100.8 78.2) (width 0.8) (layer B.Cu) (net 6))
 (segment (start 100.8 78.2) (end 106.6 84.8) (width 0.8) (layer B.Cu) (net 6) (status 20))
 (segment (start 106.6 84.8) (end 106.6 91.4) (width 0.8) (layer B.Cu) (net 6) (status 10))
 (segment (start 106.6 91.4) (end 106.6 102) (width 0.8) (layer B.Cu) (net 6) (status 10))
 (segment (start 106.6 102) (end 110.8 106.2) (width 0.8) (layer B.Cu) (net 6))
 (segment (start 110.8 106.2) (end 159.6 106.2) (width 0.8) (layer B.Cu) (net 6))
 (segment (start 159.6 106.2) (end 163.8 102) (width 0.8) (layer B.Cu) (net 6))
 (segment (start 163.8 102) (end 163.8 84.8) (width 0.8) (layer B.Cu) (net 6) (status 20))
 (segment (start 103.34 72.2) (end 103.34 72.74) (width 0.8) (layer B.Cu) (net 7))
 (segment (start 103.34 72.74) (end 105.2 74.6) (width 0.8) (layer B.Cu) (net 7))
 (segment (start 105.2 74.6) (end 107.64 74.6) (width 0.8) (layer B.Cu) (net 7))
 (segment (start 107.64 74.6) (end 113.64 68.6) (width 0.8) (layer B.Cu) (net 7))
 (segment (start 105.88 72.2) (end 105.88 69.92) (width 0.8) (layer B.Cu) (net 8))
 (segment (start 126.8 65.4) (end 130.2 68.8) (width 0.8) (layer B.Cu) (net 8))
 (segment (start 110.4 65.4) (end 126.8 65.4) (width 0.8) (layer B.Cu) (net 8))
 (segment (start 105.88 69.92) (end 110.4 65.4) (width 0.8) (layer B.Cu) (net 8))
 (segment (start 123.8 68.6) (end 127.2 72) (width 0.8) (layer B.Cu) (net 9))
 (segment (start 132.74 70.86) (end 132.74 68.8) (width 0.8) (layer B.Cu) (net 9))
 (segment (start 131.6 72) (end 132.74 70.86) (width 0.8) (layer B.Cu) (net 9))
 (segment (start 127.2 72) (end 131.6 72) (width 0.8) (layer B.Cu) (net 9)))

